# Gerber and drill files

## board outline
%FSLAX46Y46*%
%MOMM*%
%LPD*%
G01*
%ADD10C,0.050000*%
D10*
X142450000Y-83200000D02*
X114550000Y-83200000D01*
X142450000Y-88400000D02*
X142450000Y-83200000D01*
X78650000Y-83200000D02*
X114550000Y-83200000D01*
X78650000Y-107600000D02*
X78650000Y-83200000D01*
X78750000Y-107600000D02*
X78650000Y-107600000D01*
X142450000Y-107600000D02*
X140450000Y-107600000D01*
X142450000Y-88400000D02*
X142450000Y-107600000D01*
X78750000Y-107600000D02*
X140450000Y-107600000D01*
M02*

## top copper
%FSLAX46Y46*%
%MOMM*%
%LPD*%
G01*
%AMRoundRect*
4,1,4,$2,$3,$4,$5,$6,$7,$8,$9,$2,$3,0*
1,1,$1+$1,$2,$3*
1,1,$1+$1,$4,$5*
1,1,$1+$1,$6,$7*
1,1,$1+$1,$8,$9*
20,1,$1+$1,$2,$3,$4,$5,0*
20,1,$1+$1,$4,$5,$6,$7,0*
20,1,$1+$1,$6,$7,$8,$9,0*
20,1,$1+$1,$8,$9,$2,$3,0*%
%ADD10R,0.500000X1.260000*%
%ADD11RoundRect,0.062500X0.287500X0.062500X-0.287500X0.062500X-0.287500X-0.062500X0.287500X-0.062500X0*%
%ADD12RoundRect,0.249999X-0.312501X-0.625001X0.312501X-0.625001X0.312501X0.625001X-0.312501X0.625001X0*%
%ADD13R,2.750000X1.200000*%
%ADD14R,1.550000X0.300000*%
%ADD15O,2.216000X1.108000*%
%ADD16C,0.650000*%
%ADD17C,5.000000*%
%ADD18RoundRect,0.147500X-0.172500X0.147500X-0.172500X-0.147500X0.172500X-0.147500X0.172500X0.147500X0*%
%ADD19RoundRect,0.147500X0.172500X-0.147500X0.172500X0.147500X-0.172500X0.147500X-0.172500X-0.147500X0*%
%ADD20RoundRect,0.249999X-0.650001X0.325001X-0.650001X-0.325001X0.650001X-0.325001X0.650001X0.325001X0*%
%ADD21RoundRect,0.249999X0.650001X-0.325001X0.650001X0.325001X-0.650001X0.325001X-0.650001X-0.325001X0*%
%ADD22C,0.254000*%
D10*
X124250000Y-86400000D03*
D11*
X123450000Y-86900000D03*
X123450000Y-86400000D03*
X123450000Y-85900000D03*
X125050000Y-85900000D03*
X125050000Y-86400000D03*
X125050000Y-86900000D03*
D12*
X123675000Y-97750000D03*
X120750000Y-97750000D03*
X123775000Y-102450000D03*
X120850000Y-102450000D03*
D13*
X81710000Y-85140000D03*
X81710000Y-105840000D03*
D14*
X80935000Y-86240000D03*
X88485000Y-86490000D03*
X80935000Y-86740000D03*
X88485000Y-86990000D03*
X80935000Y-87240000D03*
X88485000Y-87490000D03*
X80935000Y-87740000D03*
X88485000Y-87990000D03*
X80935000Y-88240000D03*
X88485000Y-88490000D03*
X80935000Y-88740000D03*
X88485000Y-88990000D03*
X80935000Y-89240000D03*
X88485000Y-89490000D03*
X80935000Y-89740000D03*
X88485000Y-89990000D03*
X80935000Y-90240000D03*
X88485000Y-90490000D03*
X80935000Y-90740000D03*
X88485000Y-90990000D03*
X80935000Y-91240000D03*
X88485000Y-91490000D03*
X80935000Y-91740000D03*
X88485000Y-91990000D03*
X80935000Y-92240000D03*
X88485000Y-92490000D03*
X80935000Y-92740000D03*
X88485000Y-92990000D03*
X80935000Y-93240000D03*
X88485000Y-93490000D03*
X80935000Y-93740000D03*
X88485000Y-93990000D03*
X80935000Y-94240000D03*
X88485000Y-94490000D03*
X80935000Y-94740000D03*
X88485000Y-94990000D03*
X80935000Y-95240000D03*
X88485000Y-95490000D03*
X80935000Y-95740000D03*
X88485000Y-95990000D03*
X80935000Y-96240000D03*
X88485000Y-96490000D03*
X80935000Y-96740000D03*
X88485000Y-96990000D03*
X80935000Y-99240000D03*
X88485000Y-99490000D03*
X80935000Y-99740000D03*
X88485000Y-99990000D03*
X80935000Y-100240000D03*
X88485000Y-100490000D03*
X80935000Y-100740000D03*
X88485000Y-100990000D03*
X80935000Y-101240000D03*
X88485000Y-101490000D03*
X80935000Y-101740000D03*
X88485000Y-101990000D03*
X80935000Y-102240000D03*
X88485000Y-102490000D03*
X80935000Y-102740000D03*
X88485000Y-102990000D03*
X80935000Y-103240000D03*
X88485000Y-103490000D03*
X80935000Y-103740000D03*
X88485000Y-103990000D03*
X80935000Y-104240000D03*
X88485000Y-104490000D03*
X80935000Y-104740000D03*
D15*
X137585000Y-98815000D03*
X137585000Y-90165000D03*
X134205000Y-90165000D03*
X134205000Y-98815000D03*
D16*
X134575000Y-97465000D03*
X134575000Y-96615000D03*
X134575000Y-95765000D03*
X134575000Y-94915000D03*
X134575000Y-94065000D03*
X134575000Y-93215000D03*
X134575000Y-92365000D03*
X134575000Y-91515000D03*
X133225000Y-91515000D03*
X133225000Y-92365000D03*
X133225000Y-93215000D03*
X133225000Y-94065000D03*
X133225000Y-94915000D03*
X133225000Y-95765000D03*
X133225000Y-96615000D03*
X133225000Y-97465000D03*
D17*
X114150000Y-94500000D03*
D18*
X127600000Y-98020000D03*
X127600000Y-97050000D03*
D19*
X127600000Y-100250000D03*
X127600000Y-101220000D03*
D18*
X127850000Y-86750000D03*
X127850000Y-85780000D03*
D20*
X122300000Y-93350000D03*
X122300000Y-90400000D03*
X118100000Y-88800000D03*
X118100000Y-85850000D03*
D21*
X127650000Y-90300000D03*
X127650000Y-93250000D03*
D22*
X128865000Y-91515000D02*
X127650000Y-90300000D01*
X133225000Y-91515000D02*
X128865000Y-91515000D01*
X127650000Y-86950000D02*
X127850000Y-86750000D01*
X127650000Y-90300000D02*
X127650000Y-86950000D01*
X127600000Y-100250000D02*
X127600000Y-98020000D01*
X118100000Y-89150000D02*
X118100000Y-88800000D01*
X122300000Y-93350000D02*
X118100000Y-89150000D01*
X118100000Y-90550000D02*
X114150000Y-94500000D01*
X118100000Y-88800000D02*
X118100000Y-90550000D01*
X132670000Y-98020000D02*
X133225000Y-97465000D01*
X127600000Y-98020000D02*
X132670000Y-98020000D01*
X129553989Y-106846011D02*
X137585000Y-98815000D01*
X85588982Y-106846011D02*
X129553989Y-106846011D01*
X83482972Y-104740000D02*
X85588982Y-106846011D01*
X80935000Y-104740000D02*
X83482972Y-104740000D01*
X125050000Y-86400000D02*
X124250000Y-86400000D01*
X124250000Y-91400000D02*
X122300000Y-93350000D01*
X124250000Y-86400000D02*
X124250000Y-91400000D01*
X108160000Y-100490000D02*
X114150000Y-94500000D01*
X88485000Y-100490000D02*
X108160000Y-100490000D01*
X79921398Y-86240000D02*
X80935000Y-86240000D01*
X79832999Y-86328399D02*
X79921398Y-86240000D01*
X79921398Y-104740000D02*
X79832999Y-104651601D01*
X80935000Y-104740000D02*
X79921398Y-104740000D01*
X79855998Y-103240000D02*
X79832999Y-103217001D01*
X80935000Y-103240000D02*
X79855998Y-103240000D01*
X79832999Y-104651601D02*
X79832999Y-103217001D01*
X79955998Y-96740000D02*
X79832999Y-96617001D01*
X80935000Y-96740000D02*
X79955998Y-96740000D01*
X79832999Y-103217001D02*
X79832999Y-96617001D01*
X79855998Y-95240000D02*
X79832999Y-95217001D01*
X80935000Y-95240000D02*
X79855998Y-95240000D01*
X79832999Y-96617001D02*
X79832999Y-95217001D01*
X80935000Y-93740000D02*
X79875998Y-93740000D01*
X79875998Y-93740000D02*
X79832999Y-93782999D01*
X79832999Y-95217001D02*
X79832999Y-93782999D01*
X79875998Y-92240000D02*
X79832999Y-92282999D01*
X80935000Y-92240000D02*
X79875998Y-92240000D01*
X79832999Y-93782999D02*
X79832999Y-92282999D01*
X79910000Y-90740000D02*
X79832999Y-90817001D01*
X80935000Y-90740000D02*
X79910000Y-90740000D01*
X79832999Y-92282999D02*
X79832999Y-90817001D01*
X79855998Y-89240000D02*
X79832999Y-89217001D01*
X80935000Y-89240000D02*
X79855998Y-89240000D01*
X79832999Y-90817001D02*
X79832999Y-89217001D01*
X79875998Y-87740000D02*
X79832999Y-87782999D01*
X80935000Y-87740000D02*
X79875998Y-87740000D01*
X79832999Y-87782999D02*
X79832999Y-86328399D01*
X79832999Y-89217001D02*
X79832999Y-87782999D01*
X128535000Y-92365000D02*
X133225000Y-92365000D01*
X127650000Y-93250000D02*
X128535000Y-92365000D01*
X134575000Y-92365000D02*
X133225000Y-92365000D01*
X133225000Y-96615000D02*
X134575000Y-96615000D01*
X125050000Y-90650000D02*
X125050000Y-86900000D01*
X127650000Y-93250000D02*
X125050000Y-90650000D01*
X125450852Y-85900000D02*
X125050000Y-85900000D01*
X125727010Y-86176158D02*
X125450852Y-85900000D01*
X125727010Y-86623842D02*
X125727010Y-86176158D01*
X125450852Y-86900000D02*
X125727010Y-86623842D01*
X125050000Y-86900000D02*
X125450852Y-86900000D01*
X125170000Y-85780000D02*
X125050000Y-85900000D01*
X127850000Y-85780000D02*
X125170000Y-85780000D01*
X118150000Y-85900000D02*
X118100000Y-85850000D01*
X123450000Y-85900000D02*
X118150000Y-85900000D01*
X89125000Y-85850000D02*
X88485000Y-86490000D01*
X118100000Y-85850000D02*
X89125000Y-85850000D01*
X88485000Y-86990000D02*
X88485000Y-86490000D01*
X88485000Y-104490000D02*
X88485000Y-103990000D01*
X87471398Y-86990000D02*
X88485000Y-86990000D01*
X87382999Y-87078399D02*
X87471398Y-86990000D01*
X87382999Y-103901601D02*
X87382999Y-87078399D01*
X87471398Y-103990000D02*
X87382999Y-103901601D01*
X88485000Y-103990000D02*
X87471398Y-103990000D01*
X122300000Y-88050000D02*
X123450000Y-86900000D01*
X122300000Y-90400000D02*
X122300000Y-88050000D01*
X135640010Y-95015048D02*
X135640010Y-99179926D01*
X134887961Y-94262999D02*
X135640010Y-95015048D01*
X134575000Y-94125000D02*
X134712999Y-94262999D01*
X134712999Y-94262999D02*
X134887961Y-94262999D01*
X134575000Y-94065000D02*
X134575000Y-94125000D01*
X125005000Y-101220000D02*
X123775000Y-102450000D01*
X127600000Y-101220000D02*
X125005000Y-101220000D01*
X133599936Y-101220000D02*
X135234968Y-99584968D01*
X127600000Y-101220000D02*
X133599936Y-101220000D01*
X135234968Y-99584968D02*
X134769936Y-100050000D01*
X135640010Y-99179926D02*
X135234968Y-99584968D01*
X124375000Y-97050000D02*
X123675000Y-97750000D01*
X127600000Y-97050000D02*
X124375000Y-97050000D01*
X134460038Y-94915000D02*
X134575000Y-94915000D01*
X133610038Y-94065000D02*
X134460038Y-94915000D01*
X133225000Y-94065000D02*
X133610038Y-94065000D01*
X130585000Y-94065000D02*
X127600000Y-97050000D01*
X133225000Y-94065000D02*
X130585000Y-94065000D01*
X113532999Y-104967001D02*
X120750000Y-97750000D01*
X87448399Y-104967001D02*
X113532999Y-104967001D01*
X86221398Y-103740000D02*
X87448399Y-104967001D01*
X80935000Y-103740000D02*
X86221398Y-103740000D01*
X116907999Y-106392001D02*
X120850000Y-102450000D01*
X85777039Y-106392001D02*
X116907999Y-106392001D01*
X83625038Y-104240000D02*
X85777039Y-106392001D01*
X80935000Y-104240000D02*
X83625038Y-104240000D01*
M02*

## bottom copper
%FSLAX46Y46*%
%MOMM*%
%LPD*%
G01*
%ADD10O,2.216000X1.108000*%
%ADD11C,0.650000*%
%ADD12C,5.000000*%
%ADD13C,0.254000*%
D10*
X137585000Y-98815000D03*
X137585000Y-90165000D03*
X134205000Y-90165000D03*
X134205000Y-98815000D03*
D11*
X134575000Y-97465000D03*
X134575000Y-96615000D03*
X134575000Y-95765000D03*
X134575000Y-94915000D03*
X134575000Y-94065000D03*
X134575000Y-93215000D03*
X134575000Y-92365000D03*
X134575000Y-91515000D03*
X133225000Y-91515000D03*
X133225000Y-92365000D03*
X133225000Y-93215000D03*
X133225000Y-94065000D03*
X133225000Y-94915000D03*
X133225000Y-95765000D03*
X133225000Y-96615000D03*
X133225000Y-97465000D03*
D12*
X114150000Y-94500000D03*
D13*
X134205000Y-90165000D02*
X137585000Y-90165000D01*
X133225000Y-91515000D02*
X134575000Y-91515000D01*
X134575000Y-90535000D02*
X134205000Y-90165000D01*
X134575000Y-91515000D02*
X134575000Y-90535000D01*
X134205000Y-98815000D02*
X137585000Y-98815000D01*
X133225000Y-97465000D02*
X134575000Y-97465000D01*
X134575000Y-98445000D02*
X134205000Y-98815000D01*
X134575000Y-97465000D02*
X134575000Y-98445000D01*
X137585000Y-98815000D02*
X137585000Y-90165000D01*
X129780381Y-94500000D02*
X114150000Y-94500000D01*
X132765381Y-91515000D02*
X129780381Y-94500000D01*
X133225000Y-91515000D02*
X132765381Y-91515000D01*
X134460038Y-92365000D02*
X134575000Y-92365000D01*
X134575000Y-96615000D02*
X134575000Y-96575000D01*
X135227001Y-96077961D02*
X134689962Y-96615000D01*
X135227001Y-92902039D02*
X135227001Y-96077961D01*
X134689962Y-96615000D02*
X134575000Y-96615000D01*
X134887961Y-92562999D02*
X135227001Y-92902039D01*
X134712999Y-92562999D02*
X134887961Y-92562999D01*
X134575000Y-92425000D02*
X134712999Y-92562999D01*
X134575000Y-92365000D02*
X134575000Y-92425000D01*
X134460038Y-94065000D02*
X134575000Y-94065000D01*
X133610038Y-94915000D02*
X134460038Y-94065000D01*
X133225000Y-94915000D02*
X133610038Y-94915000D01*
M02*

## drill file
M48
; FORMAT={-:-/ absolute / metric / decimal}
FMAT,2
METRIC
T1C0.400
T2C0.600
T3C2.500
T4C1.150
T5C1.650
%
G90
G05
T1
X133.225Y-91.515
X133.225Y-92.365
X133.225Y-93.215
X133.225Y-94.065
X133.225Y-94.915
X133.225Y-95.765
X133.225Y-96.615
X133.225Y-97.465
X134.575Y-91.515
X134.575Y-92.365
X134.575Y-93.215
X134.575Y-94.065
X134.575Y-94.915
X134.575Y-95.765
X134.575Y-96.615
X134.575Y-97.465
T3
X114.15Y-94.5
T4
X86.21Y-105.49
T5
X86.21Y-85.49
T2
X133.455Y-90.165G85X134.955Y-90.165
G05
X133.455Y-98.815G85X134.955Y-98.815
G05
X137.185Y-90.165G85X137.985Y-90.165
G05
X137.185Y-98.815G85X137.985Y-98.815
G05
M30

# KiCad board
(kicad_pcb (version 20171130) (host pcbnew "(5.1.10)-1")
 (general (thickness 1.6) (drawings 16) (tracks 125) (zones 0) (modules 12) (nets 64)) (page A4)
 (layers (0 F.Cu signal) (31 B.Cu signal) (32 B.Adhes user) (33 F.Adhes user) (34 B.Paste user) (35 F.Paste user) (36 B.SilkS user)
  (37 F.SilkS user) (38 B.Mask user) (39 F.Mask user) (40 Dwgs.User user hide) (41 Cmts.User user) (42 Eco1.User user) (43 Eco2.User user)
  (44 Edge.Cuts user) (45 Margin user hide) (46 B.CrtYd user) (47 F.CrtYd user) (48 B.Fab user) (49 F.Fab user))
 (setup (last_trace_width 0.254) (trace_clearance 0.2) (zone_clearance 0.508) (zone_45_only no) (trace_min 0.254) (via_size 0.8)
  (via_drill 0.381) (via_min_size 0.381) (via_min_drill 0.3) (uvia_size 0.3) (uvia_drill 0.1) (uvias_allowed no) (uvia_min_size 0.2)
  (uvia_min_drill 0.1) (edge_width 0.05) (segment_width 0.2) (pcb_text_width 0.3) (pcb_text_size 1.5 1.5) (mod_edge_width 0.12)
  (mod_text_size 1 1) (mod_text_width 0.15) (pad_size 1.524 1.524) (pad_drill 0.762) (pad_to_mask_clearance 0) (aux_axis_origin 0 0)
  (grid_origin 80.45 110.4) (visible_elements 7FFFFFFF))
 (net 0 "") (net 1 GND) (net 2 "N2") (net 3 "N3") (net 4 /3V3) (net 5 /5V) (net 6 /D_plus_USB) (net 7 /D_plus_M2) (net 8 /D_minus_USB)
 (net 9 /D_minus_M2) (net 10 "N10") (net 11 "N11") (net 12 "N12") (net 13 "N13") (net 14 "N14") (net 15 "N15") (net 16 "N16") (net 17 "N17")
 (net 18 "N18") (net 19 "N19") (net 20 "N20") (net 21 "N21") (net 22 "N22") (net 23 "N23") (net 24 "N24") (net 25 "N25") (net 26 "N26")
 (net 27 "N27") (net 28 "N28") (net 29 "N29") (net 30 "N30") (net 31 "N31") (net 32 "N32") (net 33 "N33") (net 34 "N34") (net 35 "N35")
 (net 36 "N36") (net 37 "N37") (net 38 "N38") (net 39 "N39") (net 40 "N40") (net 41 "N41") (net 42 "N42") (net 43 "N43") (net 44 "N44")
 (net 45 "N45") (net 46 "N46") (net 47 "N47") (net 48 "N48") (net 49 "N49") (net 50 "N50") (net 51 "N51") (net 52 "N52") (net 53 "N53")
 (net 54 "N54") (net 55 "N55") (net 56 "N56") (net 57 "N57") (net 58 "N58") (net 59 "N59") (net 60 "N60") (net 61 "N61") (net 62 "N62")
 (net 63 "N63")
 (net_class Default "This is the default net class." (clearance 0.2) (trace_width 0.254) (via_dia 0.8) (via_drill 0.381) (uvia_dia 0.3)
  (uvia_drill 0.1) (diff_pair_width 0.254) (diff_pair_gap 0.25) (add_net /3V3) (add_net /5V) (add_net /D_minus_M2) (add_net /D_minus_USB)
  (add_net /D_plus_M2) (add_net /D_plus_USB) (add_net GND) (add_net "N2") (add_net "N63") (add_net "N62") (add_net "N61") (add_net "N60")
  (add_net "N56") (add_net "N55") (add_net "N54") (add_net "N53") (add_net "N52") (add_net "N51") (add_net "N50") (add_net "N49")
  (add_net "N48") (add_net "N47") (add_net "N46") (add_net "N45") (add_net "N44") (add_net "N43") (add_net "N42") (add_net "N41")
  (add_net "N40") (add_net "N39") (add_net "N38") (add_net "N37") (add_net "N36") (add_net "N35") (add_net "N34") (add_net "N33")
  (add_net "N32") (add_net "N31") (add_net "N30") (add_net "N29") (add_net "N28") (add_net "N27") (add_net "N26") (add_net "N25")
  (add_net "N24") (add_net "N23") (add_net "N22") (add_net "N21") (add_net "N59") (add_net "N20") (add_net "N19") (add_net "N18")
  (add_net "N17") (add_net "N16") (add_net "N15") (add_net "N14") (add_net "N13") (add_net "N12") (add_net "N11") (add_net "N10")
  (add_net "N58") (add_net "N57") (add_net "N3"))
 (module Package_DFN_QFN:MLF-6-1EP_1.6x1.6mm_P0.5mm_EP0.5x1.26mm (layer F.Cu) (at 124.25 86.4 180)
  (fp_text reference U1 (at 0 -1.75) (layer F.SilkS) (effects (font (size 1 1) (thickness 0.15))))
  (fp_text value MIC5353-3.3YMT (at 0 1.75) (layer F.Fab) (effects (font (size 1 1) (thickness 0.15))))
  (pad "" smd roundrect (at 0 0.315 180) (size 0.4 0.51) (layers F.Paste) (roundrect_rratio 0.25))
  (pad "" smd roundrect (at 0 -0.315 180) (size 0.4 0.51) (layers F.Paste) (roundrect_rratio 0.25))
  (pad 7 smd rect (at 0 0 180) (size 0.5 1.26) (layers F.Cu F.Mask) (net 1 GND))
  (pad 6 smd roundrect (at 0.8 -0.5 180) (size 0.7 0.25) (layers F.Cu F.Paste F.Mask) (roundrect_rratio 0.25) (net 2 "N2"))
  (pad 5 smd roundrect (at 0.8 0 180) (size 0.7 0.25) (layers F.Cu F.Paste F.Mask) (roundrect_rratio 0.25) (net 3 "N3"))
  (pad 4 smd roundrect (at 0.8 0.5 180) (size 0.7 0.25) (layers F.Cu F.Paste F.Mask) (roundrect_rratio 0.25) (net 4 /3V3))
  (pad 3 smd roundrect (at -0.8 0.5 180) (size 0.7 0.25) (layers F.Cu F.Paste F.Mask) (roundrect_rratio 0.25) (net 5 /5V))
  (pad 2 smd roundrect (at -0.8 0 180) (size 0.7 0.25) (layers F.Cu F.Paste F.Mask) (roundrect_rratio 0.25) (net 1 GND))
  (pad 1 smd roundrect (at -0.8 -0.5 180) (size 0.7 0.25) (layers F.Cu F.Paste F.Mask) (roundrect_rratio 0.25) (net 5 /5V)))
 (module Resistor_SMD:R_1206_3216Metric (layer F.Cu) (at 122.2125 97.75)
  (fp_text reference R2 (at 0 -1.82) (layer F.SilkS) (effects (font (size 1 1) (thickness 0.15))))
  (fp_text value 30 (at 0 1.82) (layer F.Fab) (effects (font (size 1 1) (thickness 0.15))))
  (pad 2 smd roundrect (at 1.4625 0) (size 1.125 1.75) (layers F.Cu F.Paste F.Mask) (roundrect_rratio 0.2222213333333333)
   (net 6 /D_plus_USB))
  (pad 1 smd roundrect (at -1.4625 0) (size 1.125 1.75) (layers F.Cu F.Paste F.Mask) (roundrect_rratio 0.2222213333333333)
   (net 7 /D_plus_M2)))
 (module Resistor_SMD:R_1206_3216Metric (layer F.Cu) (at 122.3125 102.45)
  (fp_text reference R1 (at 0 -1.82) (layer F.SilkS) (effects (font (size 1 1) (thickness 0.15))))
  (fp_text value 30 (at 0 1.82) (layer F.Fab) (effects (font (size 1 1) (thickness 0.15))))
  (pad 2 smd roundrect (at 1.4625 0) (size 1.125 1.75) (layers F.Cu F.Paste F.Mask) (roundrect_rratio 0.2222213333333333)
   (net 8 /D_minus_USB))
  (pad 1 smd roundrect (at -1.4625 0) (size 1.125 1.75) (layers F.Cu F.Paste F.Mask) (roundrect_rratio 0.2222213333333333)
   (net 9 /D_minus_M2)))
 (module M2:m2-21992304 (layer F.Cu) (at 84.56 95.49 90)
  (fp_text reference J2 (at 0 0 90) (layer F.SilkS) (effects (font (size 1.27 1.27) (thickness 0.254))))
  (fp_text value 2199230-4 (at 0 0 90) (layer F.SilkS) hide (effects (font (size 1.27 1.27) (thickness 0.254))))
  (pad MP2 smd rect (at 10.35 -2.85 90) (size 1.2 2.75) (layers F.Cu F.Paste F.Mask))
  (pad MP1 smd rect (at -10.35 -2.85 90) (size 1.2 2.75) (layers F.Cu F.Paste F.Mask))
  (pad MH2 np_thru_hole circle (at 10 1.65 90) (size 1.65 0) (drill 1.65) (layers *.Cu *.Mask))
  (pad MH1 np_thru_hole circle (at -10 1.65 90) (size 1.15 0) (drill 1.15) (layers *.Cu *.Mask))
  (pad 75 smd rect (at 9.25 -3.625 90) (size 0.3 1.55) (layers F.Cu F.Paste F.Mask) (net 1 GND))
  (pad 74 smd rect (at 9 3.925 90) (size 0.3 1.55) (layers F.Cu F.Paste F.Mask) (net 4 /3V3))
  (pad 73 smd rect (at 8.75 -3.625 90) (size 0.3 1.55) (layers F.Cu F.Paste F.Mask) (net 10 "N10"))
  (pad 72 smd rect (at 8.5 3.925 90) (size 0.3 1.55) (layers F.Cu F.Paste F.Mask) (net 4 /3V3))
  (pad 71 smd rect (at 8.25 -3.625 90) (size 0.3 1.55) (layers F.Cu F.Paste F.Mask) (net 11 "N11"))
  (pad 70 smd rect (at 8 3.925 90) (size 0.3 1.55) (layers F.Cu F.Paste F.Mask) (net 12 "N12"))
  (pad 69 smd rect (at 7.75 -3.625 90) (size 0.3 1.55) (layers F.Cu F.Paste F.Mask) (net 1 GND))
  (pad 68 smd rect (at 7.5 3.925 90) (size 0.3 1.55) (layers F.Cu F.Paste F.Mask) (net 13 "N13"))
  (pad 67 smd rect (at 7.25 -3.625 90) (size 0.3 1.55) (layers F.Cu F.Paste F.Mask) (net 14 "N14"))
  (pad 66 smd rect (at 7 3.925 90) (size 0.3 1.55) (layers F.Cu F.Paste F.Mask) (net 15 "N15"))
  (pad 65 smd rect (at 6.75 -3.625 90) (size 0.3 1.55) (layers F.Cu F.Paste F.Mask) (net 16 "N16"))
  (pad 64 smd rect (at 6.5 3.925 90) (size 0.3 1.55) (layers F.Cu F.Paste F.Mask) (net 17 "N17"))
  (pad 63 smd rect (at 6.25 -3.625 90) (size 0.3 1.55) (layers F.Cu F.Paste F.Mask) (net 1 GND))
  (pad 62 smd rect (at 6 3.925 90) (size 0.3 1.55) (layers F.Cu F.Paste F.Mask) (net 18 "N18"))
  (pad 61 smd rect (at 5.75 -3.625 90) (size 0.3 1.55) (layers F.Cu F.Paste F.Mask) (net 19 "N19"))
  (pad 60 smd rect (at 5.5 3.925 90) (size 0.3 1.55) (layers F.Cu F.Paste F.Mask) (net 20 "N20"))
  (pad 59 smd rect (at 5.25 -3.625 90) (size 0.3 1.55) (layers F.Cu F.Paste F.Mask) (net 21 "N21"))
  (pad 58 smd rect (at 5 3.925 90) (size 0.3 1.55) (layers F.Cu F.Paste F.Mask) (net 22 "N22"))
  (pad 57 smd rect (at 4.75 -3.625 90) (size 0.3 1.55) (layers F.Cu F.Paste F.Mask) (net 1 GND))
  (pad 56 smd rect (at 4.5 3.925 90) (size 0.3 1.55) (layers F.Cu F.Paste F.Mask) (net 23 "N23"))
  (pad 55 smd rect (at 4.25 -3.625 90) (size 0.3 1.55) (layers F.Cu F.Paste F.Mask) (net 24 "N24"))
  (pad 54 smd rect (at 4 3.925 90) (size 0.3 1.55) (layers F.Cu F.Paste F.Mask) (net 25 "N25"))
  (pad 53 smd rect (at 3.75 -3.625 90) (size 0.3 1.55) (layers F.Cu F.Paste F.Mask) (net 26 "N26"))
  (pad 52 smd rect (at 3.5 3.925 90) (size 0.3 1.55) (layers F.Cu F.Paste F.Mask) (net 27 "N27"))
  (pad 51 smd rect (at 3.25 -3.625 90) (size 0.3 1.55) (layers F.Cu F.Paste F.Mask) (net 1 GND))
  (pad 50 smd rect (at 3 3.925 90) (size 0.3 1.55) (layers F.Cu F.Paste F.Mask) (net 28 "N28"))
  (pad 49 smd rect (at 2.75 -3.625 90) (size 0.3 1.55) (layers F.Cu F.Paste F.Mask) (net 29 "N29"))
  (pad 48 smd rect (at 2.5 3.925 90) (size 0.3 1.55) (layers F.Cu F.Paste F.Mask) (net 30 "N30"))
  (pad 47 smd rect (at 2.25 -3.625 90) (size 0.3 1.55) (layers F.Cu F.Paste F.Mask) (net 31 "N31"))
  (pad 46 smd rect (at 2 3.925 90) (size 0.3 1.55) (layers F.Cu F.Paste F.Mask) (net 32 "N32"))
  (pad 45 smd rect (at 1.75 -3.625 90) (size 0.3 1.55) (layers F.Cu F.Paste F.Mask) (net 1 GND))
  (pad 44 smd rect (at 1.5 3.925 90) (size 0.3 1.55) (layers F.Cu F.Paste F.Mask) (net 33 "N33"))
  (pad 43 smd rect (at 1.25 -3.625 90) (size 0.3 1.55) (layers F.Cu F.Paste F.Mask) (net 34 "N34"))
  (pad 42 smd rect (at 1 3.925 90) (size 0.3 1.55) (layers F.Cu F.Paste F.Mask) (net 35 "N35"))
  (pad 41 smd rect (at 0.75 -3.625 90) (size 0.3 1.55) (layers F.Cu F.Paste F.Mask) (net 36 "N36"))
  (pad 40 smd rect (at 0.5 3.925 90) (size 0.3 1.55) (layers F.Cu F.Paste F.Mask) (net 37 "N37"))
  (pad 39 smd rect (at 0.25 -3.625 90) (size 0.3 1.55) (layers F.Cu F.Paste F.Mask) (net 1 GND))
  (pad 38 smd rect (at 0 3.925 90) (size 0.3 1.55) (layers F.Cu F.Paste F.Mask) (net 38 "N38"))
  (pad 37 smd rect (at -0.25 -3.625 90) (size 0.3 1.55) (layers F.Cu F.Paste F.Mask) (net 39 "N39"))
  (pad 36 smd rect (at -0.5 3.925 90) (size 0.3 1.55) (layers F.Cu F.Paste F.Mask) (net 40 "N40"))
  (pad 35 smd rect (at -0.75 -3.625 90) (size 0.3 1.55) (layers F.Cu F.Paste F.Mask) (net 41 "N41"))
  (pad 34 smd rect (at -1 3.925 90) (size 0.3 1.55) (layers F.Cu F.Paste F.Mask) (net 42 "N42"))
  (pad 33 smd rect (at -1.25 -3.625 90) (size 0.3 1.55) (layers F.Cu F.Paste F.Mask) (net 1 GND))
  (pad 32 smd rect (at -1.5 3.925 90) (size 0.3 1.55) (layers F.Cu F.Paste F.Mask) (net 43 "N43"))
  (pad 23 smd rect (at -3.75 -3.625 90) (size 0.3 1.55) (layers F.Cu F.Paste F.Mask) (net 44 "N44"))
  (pad 22 smd rect (at -4 3.925 90) (size 0.3 1.55) (layers F.Cu F.Paste F.Mask) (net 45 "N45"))
  (pad 21 smd rect (at -4.25 -3.625 90) (size 0.3 1.55) (layers F.Cu F.Paste F.Mask) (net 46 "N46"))
  (pad 20 smd rect (at -4.5 3.925 90) (size 0.3 1.55) (layers F.Cu F.Paste F.Mask) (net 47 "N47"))
  (pad 19 smd rect (at -4.75 -3.625 90) (size 0.3 1.55) (layers F.Cu F.Paste F.Mask) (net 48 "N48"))
  (pad 18 smd rect (at -5 3.925 90) (size 0.3 1.55) (layers F.Cu F.Paste F.Mask) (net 1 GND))
  (pad 17 smd rect (at -5.25 -3.625 90) (size 0.3 1.55) (layers F.Cu F.Paste F.Mask) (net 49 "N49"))
  (pad 16 smd rect (at -5.5 3.925 90) (size 0.3 1.55) (layers F.Cu F.Paste F.Mask) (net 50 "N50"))
  (pad 15 smd rect (at -5.75 -3.625 90) (size 0.3 1.55) (layers F.Cu F.Paste F.Mask) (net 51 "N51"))
  (pad 14 smd rect (at -6 3.925 90) (size 0.3 1.55) (layers F.Cu F.Paste F.Mask) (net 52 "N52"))
  (pad 13 smd rect (at -6.25 -3.625 90) (size 0.3 1.55) (layers F.Cu F.Paste F.Mask) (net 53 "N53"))
  (pad 12 smd rect (at -6.5 3.925 90) (size 0.3 1.55) (layers F.Cu F.Paste F.Mask) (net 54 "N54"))
  (pad 11 smd rect (at -6.75 -3.625 90) (size 0.3 1.55) (layers F.Cu F.Paste F.Mask) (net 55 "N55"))
  (pad 10 smd rect (at -7 3.925 90) (size 0.3 1.55) (layers F.Cu F.Paste F.Mask) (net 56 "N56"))
  (pad 9 smd rect (at -7.25 -3.625 90) (size 0.3 1.55) (layers F.Cu F.Paste F.Mask) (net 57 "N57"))
  (pad 8 smd rect (at -7.5 3.925 90) (size 0.3 1.55) (layers F.Cu F.Paste F.Mask) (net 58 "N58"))
  (pad 7 smd rect (at -7.75 -3.625 90) (size 0.3 1.55) (layers F.Cu F.Paste F.Mask) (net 1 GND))
  (pad 6 smd rect (at -8 3.925 90) (size 0.3 1.55) (layers F.Cu F.Paste F.Mask) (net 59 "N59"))
  (pad 5 smd rect (at -8.25 -3.625 90) (size 0.3 1.55) (layers F.Cu F.Paste F.Mask) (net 7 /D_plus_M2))
  (pad 4 smd rect (at -8.5 3.925 90) (size 0.3 1.55) (layers F.Cu F.Paste F.Mask) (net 4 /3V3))
  (pad 3 smd rect (at -8.75 -3.625 90) (size 0.3 1.55) (layers F.Cu F.Paste F.Mask) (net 9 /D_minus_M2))
  (pad 2 smd rect (at -9 3.925 90) (size 0.3 1.55) (layers F.Cu F.Paste F.Mask) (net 4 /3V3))
  (pad 1 smd rect (at -9.25 -3.625 90) (size 0.3 1.55) (layers F.Cu F.Paste F.Mask) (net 1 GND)))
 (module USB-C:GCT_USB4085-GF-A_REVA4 (layer F.Cu) (at 137.25 94.49 90)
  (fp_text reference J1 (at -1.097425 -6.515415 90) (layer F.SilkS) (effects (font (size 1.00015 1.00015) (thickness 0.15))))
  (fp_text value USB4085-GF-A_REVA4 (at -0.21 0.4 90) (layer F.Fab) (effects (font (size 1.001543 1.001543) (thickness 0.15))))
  (pad P4 thru_hole oval (at -4.325 0.335 90) (size 1.108 2.216) (drill oval 0.6 1.4) (layers *.Cu *.Mask) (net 1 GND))
  (pad P3 thru_hole oval (at 4.325 0.335 90) (size 1.108 2.216) (drill oval 0.6 1.4) (layers *.Cu *.Mask) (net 1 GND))
  (pad P2 thru_hole oval (at 4.325 -3.045 90) (size 1.108 2.216) (drill oval 0.6 2.1) (layers *.Cu *.Mask) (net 1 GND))
  (pad P1 thru_hole oval (at -4.325 -3.045 90) (size 1.108 2.216) (drill oval 0.6 2.1) (layers *.Cu *.Mask) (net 1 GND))
  (pad B12 thru_hole circle (at -2.975 -2.675 90) (size 0.65 0.65) (drill 0.4) (layers *.Cu *.Mask) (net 1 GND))
  (pad B9 thru_hole circle (at -2.125 -2.675 90) (size 0.65 0.65) (drill 0.4) (layers *.Cu *.Mask) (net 5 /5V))
  (pad B8 thru_hole circle (at -1.275 -2.675 90) (size 0.65 0.65) (drill 0.4) (layers *.Cu *.Mask) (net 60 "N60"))
  (pad B7 thru_hole circle (at -0.425 -2.675 90) (size 0.65 0.65) (drill 0.4) (layers *.Cu *.Mask) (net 6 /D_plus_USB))
  (pad B6 thru_hole circle (at 0.425 -2.675 90) (size 0.65 0.65) (drill 0.4) (layers *.Cu *.Mask) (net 8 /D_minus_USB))
  (pad B5 thru_hole circle (at 1.275 -2.675 90) (size 0.65 0.65) (drill 0.4) (layers *.Cu *.Mask) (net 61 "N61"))
  (pad B4 thru_hole circle (at 2.125 -2.675 90) (size 0.65 0.65) (drill 0.4) (layers *.Cu *.Mask) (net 5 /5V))
  (pad B1 thru_hole circle (at 2.975 -2.675 90) (size 0.65 0.65) (drill 0.4) (layers *.Cu *.Mask) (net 1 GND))
  (pad A12 thru_hole circle (at 2.975 -4.025 90) (size 0.65 0.65) (drill 0.4) (layers *.Cu *.Mask) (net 1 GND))
  (pad A9 thru_hole circle (at 2.125 -4.025 90) (size 0.65 0.65) (drill 0.4) (layers *.Cu *.Mask) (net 5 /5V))
  (pad A8 thru_hole circle (at 1.275 -4.025 90) (size 0.65 0.65) (drill 0.4) (layers *.Cu *.Mask) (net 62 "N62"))
  (pad A7 thru_hole circle (at 0.425 -4.025 90) (size 0.65 0.65) (drill 0.4) (layers *.Cu *.Mask) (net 6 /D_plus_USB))
  (pad A6 thru_hole circle (at -0.425 -4.025 90) (size 0.65 0.65) (drill 0.4) (layers *.Cu *.Mask) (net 8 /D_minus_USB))
  (pad A5 thru_hole circle (at -1.275 -4.025 90) (size 0.65 0.65) (drill 0.4) (layers *.Cu *.Mask) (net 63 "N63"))
  (pad A4 thru_hole circle (at -2.125 -4.025 90) (size 0.65 0.65) (drill 0.4) (layers *.Cu *.Mask) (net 5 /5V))
  (pad A1 thru_hole circle (at -2.975 -4.025 90) (size 0.65 0.65) (drill 0.4) (layers *.Cu *.Mask) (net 1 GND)))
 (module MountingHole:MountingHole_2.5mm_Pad (layer F.Cu) (at 114.15 94.5)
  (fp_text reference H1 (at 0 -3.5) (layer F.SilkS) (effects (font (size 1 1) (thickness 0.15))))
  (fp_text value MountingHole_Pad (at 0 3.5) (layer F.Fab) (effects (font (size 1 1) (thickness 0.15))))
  (pad 1 thru_hole circle (at 0 0) (size 5 5) (drill 2.5) (layers *.Cu *.Mask) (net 1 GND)))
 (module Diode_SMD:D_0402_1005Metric (layer F.Cu) (at 127.6 97.535 270)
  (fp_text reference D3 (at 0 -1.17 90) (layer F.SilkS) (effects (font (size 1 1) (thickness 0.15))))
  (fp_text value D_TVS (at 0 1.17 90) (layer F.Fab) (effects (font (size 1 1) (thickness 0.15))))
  (pad 2 smd roundrect (at 0.485 0 270) (size 0.59 0.64) (layers F.Cu F.Paste F.Mask) (roundrect_rratio 0.25) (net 1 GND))
  (pad 1 smd roundrect (at -0.485 0 270) (size 0.59 0.64) (layers F.Cu F.Paste F.Mask) (roundrect_rratio 0.25) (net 6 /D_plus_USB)))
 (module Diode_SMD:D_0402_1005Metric (layer F.Cu) (at 127.6 100.735 90)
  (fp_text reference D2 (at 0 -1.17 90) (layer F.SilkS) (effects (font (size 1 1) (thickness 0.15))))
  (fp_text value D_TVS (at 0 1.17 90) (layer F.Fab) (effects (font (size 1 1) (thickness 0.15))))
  (pad 2 smd roundrect (at 0.485 0 90) (size 0.59 0.64) (layers F.Cu F.Paste F.Mask) (roundrect_rratio 0.25) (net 1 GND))
  (pad 1 smd roundrect (at -0.485 0 90) (size 0.59 0.64) (layers F.Cu F.Paste F.Mask) (roundrect_rratio 0.25) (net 8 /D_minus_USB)))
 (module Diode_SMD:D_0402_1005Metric (layer F.Cu) (at 127.85 86.265 270)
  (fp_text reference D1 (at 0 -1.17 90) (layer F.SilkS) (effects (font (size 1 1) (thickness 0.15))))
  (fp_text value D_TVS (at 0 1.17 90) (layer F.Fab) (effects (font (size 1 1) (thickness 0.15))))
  (pad 2 smd roundrect (at 0.485 0 270) (size 0.59 0.64) (layers F.Cu F.Paste F.Mask) (roundrect_rratio 0.25) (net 1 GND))
  (pad 1 smd roundrect (at -0.485 0 270) (size 0.59 0.64) (layers F.Cu F.Paste F.Mask) (roundrect_rratio 0.25) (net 5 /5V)))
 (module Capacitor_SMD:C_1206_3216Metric (layer F.Cu) (at 122.3 91.875 270)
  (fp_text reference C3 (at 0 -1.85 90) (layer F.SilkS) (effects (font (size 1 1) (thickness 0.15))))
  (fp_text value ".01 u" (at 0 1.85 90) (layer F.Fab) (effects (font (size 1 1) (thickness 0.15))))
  (pad 2 smd roundrect (at 1.475 0 270) (size 1.15 1.8) (layers F.Cu F.Paste F.Mask) (roundrect_rratio 0.2173904347826087) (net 1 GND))
  (pad 1 smd roundrect (at -1.475 0 270) (size 1.15 1.8) (layers F.Cu F.Paste F.Mask) (roundrect_rratio 0.2173904347826087) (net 2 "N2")))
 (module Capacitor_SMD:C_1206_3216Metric (layer F.Cu) (at 118.1 87.325 270)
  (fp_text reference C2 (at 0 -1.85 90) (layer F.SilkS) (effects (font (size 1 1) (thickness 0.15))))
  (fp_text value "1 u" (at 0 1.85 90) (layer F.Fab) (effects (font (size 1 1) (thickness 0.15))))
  (pad 2 smd roundrect (at 1.475 0 270) (size 1.15 1.8) (layers F.Cu F.Paste F.Mask) (roundrect_rratio 0.2173904347826087) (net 1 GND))
  (pad 1 smd roundrect (at -1.475 0 270) (size 1.15 1.8) (layers F.Cu F.Paste F.Mask) (roundrect_rratio 0.2173904347826087) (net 4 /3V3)))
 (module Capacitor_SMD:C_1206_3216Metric (layer F.Cu) (at 127.65 91.775 90)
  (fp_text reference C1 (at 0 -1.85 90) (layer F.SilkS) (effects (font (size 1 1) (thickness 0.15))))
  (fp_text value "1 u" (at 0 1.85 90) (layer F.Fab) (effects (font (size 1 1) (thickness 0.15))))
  (pad 2 smd roundrect (at 1.475 0 90) (size 1.15 1.8) (layers F.Cu F.Paste F.Mask) (roundrect_rratio 0.2173904347826087) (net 1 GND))
  (pad 1 smd roundrect (at -1.475 0 90) (size 1.15 1.8) (layers F.Cu F.Paste F.Mask) (roundrect_rratio 0.2173904347826087) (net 5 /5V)))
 (gr_line (start 142.45 83.2) (end 114.55 83.2) (layer Edge.Cuts) (width 0.05))
 (gr_line (start 142.45 88.4) (end 142.45 83.2) (layer Edge.Cuts) (width 0.05))
 (gr_line (start 78.65 83.2) (end 114.55 83.2) (layer Edge.Cuts) (width 0.05))
 (gr_line (start 78.65 107.6) (end 78.65 83.2) (layer Edge.Cuts) (width 0.05))
 (gr_line (start 78.75 107.6) (end 78.65 107.6) (layer Edge.Cuts) (width 0.05))
 (gr_line (start 142.45 107.6) (end 140.45 107.6) (layer Edge.Cuts) (width 0.05))
 (gr_line (start 142.45 88.4) (end 142.45 107.6) (layer Edge.Cuts) (width 0.05))
 (gr_line (start 78.75 107.6) (end 140.45 107.6) (layer Edge.Cuts) (width 0.05))
 (segment (start 134.205 90.165) (end 137.585 90.165) (width 0.254) (layer B.Cu) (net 1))
 (segment (start 133.225 91.515) (end 134.575 91.515) (width 0.254) (layer B.Cu) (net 1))
 (segment (start 134.575 90.535) (end 134.205 90.165) (width 0.254) (layer B.Cu) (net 1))
 (segment (start 134.575 91.515) (end 134.575 90.535) (width 0.254) (layer B.Cu) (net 1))
 (segment (start 134.205 98.815) (end 137.585 98.815) (width 0.254) (layer B.Cu) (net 1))
 (segment (start 133.225 97.465) (end 134.575 97.465) (width 0.254) (layer B.Cu) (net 1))
 (segment (start 134.575 98.445) (end 134.205 98.815) (width 0.254) (layer B.Cu) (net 1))
 (segment (start 134.575 97.465) (end 134.575 98.445) (width 0.254) (layer B.Cu) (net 1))
 (segment (start 137.585 98.815) (end 137.585 90.165) (width 0.254) (layer B.Cu) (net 1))
 (segment (start 128.865 91.515) (end 127.65 90.3) (width 0.254) (layer F.Cu) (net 1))
 (segment (start 133.225 91.515) (end 128.865 91.515) (width 0.254) (layer F.Cu) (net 1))
 (segment (start 127.65 86.95) (end 127.85 86.75) (width 0.254) (layer F.Cu) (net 1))
 (segment (start 127.65 90.3) (end 127.65 86.95) (width 0.254) (layer F.Cu) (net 1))
 (segment (start 127.6 100.25) (end 127.6 98.02) (width 0.254) (layer F.Cu) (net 1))
 (segment (start 118.1 89.15) (end 118.1 88.8) (width 0.254) (layer F.Cu) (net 1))
 (segment (start 122.3 93.35) (end 118.1 89.15) (width 0.254) (layer F.Cu) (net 1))
 (segment (start 118.1 90.55) (end 114.15 94.5) (width 0.254) (layer F.Cu) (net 1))
 (segment (start 118.1 88.8) (end 118.1 90.55) (width 0.254) (layer F.Cu) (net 1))
 (segment (start 132.67 98.02) (end 133.225 97.465) (width 0.254) (layer F.Cu) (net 1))
 (segment (start 127.6 98.02) (end 132.67 98.02) (width 0.254) (layer F.Cu) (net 1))
 (segment (start 129.553989 106.846011) (end 137.585 98.815) (width 0.254) (layer F.Cu) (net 1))
 (segment (start 85.588982 106.846011) (end 129.553989 106.846011) (width 0.254) (layer F.Cu) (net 1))
 (segment (start 83.482972 104.74) (end 85.588982 106.846011) (width 0.254) (layer F.Cu) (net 1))
 (segment (start 80.935 104.74) (end 83.482972 104.74) (width 0.254) (layer F.Cu) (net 1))
 (segment (start 125.05 86.4) (end 124.25 86.4) (width 0.254) (layer F.Cu) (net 1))
 (segment (start 124.25 91.4) (end 122.3 93.35) (width 0.254) (layer F.Cu) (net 1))
 (segment (start 124.25 86.4) (end 124.25 91.4) (width 0.254) (layer F.Cu) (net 1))
 (segment (start 108.16 100.49) (end 114.15 94.5) (width 0.254) (layer F.Cu) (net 1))
 (segment (start 88.485 100.49) (end 108.16 100.49) (width 0.254) (layer F.Cu) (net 1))
 (segment (start 79.921398 86.24) (end 80.935 86.24) (width 0.254) (layer F.Cu) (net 1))
 (segment (start 79.832999 86.328399) (end 79.921398 86.24) (width 0.254) (layer F.Cu) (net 1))
 (segment (start 79.921398 104.74) (end 79.832999 104.651601) (width 0.254) (layer F.Cu) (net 1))
 (segment (start 80.935 104.74) (end 79.921398 104.74) (width 0.254) (layer F.Cu) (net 1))
 (segment (start 79.855998 103.24) (end 79.832999 103.217001) (width 0.254) (layer F.Cu) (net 1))
 (segment (start 80.935 103.24) (end 79.855998 103.24) (width 0.254) (layer F.Cu) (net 1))
 (segment (start 79.832999 104.651601) (end 79.832999 103.217001) (width 0.254) (layer F.Cu) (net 1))
 (segment (start 79.955998 96.74) (end 79.832999 96.617001) (width 0.254) (layer F.Cu) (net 1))
 (segment (start 80.935 96.74) (end 79.955998 96.74) (width 0.254) (layer F.Cu) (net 1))
 (segment (start 79.832999 103.217001) (end 79.832999 96.617001) (width 0.254) (layer F.Cu) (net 1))
 (segment (start 79.855998 95.24) (end 79.832999 95.217001) (width 0.254) (layer F.Cu) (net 1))
 (segment (start 80.935 95.24) (end 79.855998 95.24) (width 0.254) (layer F.Cu) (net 1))
 (segment (start 79.832999 96.617001) (end 79.832999 95.217001) (width 0.254) (layer F.Cu) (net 1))
 (segment (start 80.935 93.74) (end 79.875998 93.74) (width 0.254) (layer F.Cu) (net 1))
 (segment (start 79.875998 93.74) (end 79.832999 93.782999) (width 0.254) (layer F.Cu) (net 1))
 (segment (start 79.832999 95.217001) (end 79.832999 93.782999) (width 0.254) (layer F.Cu) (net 1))
 (segment (start 79.875998 92.24) (end 79.832999 92.282999) (width 0.254) (layer F.Cu) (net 1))
 (segment (start 80.935 92.24) (end 79.875998 92.24) (width 0.254) (layer F.Cu) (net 1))
 (segment (start 79.832999 93.782999) (end 79.832999 92.282999) (width 0.254) (layer F.Cu) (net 1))
 (segment (start 79.91 90.74) (end 79.832999 90.817001) (width 0.254) (layer F.Cu) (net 1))
 (segment (start 80.935 90.74) (end 79.91 90.74) (width 0.254) (layer F.Cu) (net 1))
 (segment (start 79.832999 92.282999) (end 79.832999 90.817001) (width 0.254) (layer F.Cu) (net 1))
 (segment (start 79.855998 89.24) (end 79.832999 89.217001) (width 0.254) (layer F.Cu) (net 1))
 (segment (start 80.935 89.24) (end 79.855998 89.24) (width 0.254) (layer F.Cu) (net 1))
 (segment (start 79.832999 90.817001) (end 79.832999 89.217001) (width 0.254) (layer F.Cu) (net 1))
 (segment (start 79.875998 87.74) (end 79.832999 87.782999) (width 0.254) (layer F.Cu) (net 1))
 (segment (start 80.935 87.74) (end 79.875998 87.74) (width 0.254) (layer F.Cu) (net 1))
 (segment (start 79.832999 87.782999) (end 79.832999 86.328399) (width 0.254) (layer F.Cu) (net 1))
 (segment (start 79.832999 89.217001) (end 79.832999 87.782999) (width 0.254) (layer F.Cu) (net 1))
 (segment (start 129.780381 94.5) (end 114.15 94.5) (width 0.254) (layer B.Cu) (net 1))
 (segment (start 132.765381 91.515) (end 129.780381 94.5) (width 0.254) (layer B.Cu) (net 1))
 (segment (start 133.225 91.515) (end 132.765381 91.515) (width 0.254) (layer B.Cu) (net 1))
 (segment (start 128.535 92.365) (end 133.225 92.365) (width 0.254) (layer F.Cu) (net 5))
 (segment (start 127.65 93.25) (end 128.535 92.365) (width 0.254) (layer F.Cu) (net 5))
 (segment (start 134.575 92.365) (end 133.225 92.365) (width 0.254) (layer F.Cu) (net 5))
 (segment (start 133.225 96.615) (end 134.575 96.615) (width 0.254) (layer F.Cu) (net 5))
 (segment (start 134.460038 92.365) (end 134.575 92.365) (width 0.254) (layer B.Cu) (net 5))
 (segment (start 134.575 96.615) (end 134.575 96.575) (width 0.254) (layer B.Cu) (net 5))
 (segment (start 125.05 90.65) (end 125.05 86.9) (width 0.254) (layer F.Cu) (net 5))
 (segment (start 127.65 93.25) (end 125.05 90.65) (width 0.254) (layer F.Cu) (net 5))
 (segment (start 125.450852 85.9) (end 125.05 85.9) (width 0.254) (layer F.Cu) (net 5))
 (segment (start 125.72701 86.176158) (end 125.450852 85.9) (width 0.254) (layer F.Cu) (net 5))
 (segment (start 125.72701 86.623842) (end 125.72701 86.176158) (width 0.254) (layer F.Cu) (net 5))
 (segment (start 125.450852 86.9) (end 125.72701 86.623842) (width 0.254) (layer F.Cu) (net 5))
 (segment (start 125.05 86.9) (end 125.450852 86.9) (width 0.254) (layer F.Cu) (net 5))
 (segment (start 125.17 85.78) (end 125.05 85.9) (width 0.254) (layer F.Cu) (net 5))
 (segment (start 127.85 85.78) (end 125.17 85.78) (width 0.254) (layer F.Cu) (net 5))
 (segment (start 135.227001 96.077961) (end 134.689962 96.615) (width 0.254) (layer B.Cu) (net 5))
 (segment (start 135.227001 92.902039) (end 135.227001 96.077961) (width 0.254) (layer B.Cu) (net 5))
 (segment (start 134.689962 96.615) (end 134.575 96.615) (width 0.254) (layer B.Cu) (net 5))
 (segment (start 134.887961 92.562999) (end 135.227001 92.902039) (width 0.254) (layer B.Cu) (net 5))
 (segment (start 134.712999 92.562999) (end 134.887961 92.562999) (width 0.254) (layer B.Cu) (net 5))
 (segment (start 134.575 92.425) (end 134.712999 92.562999) (width 0.254) (layer B.Cu) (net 5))
 (segment (start 134.575 92.365) (end 134.575 92.425) (width 0.254) (layer B.Cu) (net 5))
 (segment (start 118.15 85.9) (end 118.1 85.85) (width 0.254) (layer F.Cu) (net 4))
 (segment (start 123.45 85.9) (end 118.15 85.9) (width 0.254) (layer F.Cu) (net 4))
 (segment (start 89.125 85.85) (end 88.485 86.49) (width 0.254) (layer F.Cu) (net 4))
 (segment (start 118.1 85.85) (end 89.125 85.85) (width 0.254) (layer F.Cu) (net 4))
 (segment (start 88.485 86.99) (end 88.485 86.49) (width 0.254) (layer F.Cu) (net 4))
 (segment (start 88.485 104.49) (end 88.485 103.99) (width 0.254) (layer F.Cu) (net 4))
 (segment (start 87.471398 86.99) (end 88.485 86.99) (width 0.254) (layer F.Cu) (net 4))
 (segment (start 87.382999 87.078399) (end 87.471398 86.99) (width 0.254) (layer F.Cu) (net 4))
 (segment (start 87.382999 103.901601) (end 87.382999 87.078399) (width 0.254) (layer F.Cu) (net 4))
 (segment (start 87.471398 103.99) (end 87.382999 103.901601) (width 0.254) (layer F.Cu) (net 4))
 (segment (start 88.485 103.99) (end 87.471398 103.99) (width 0.254) (layer F.Cu) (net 4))
 (segment (start 122.3 88.05) (end 123.45 86.9) (width 0.254) (layer F.Cu) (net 2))
 (segment (start 122.3 90.4) (end 122.3 88.05) (width 0.254) (layer F.Cu) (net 2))
 (segment (start 134.460038 94.065) (end 134.575 94.065) (width 0.254) (layer B.Cu) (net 8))
 (segment (start 133.610038 94.915) (end 134.460038 94.065) (width 0.254) (layer B.Cu) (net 8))
 (segment (start 133.225 94.915) (end 133.610038 94.915) (width 0.254) (layer B.Cu) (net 8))
 (segment (start 135.64001 95.015048) (end 135.64001 99.179926) (width 0.254) (layer F.Cu) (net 8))
 (segment (start 134.887961 94.262999) (end 135.64001 95.015048) (width 0.254) (layer F.Cu) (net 8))
 (segment (start 134.575 94.125) (end 134.712999 94.262999) (width 0.254) (layer F.Cu) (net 8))
 (segment (start 134.712999 94.262999) (end 134.887961 94.262999) (width 0.254) (layer F.Cu) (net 8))
 (segment (start 134.575 94.065) (end 134.575 94.125) (width 0.254) (layer F.Cu) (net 8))
 (segment (start 125.005 101.22) (end 123.775 102.45) (width 0.254) (layer F.Cu) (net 8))
 (segment (start 127.6 101.22) (end 125.005 101.22) (width 0.254) (layer F.Cu) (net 8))
 (segment (start 133.599936 101.22) (end 135.234968 99.584968) (width 0.254) (layer F.Cu) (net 8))
 (segment (start 127.6 101.22) (end 133.599936 101.22) (width 0.254) (layer F.Cu) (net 8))
 (segment (start 135.234968 99.584968) (end 134.769936 100.05) (width 0.254) (layer F.Cu) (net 8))
 (segment (start 135.64001 99.179926) (end 135.234968 99.584968) (width 0.254) (layer F.Cu) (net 8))
 (segment (start 124.375 97.05) (end 123.675 97.75) (width 0.254) (layer F.Cu) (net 6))
 (segment (start 127.6 97.05) (end 124.375 97.05) (width 0.254) (layer F.Cu) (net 6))
 (segment (start 134.460038 94.915) (end 134.575 94.915) (width 0.254) (layer F.Cu) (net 6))
 (segment (start 133.610038 94.065) (end 134.460038 94.915) (width 0.254) (layer F.Cu) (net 6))
 (segment (start 133.225 94.065) (end 133.610038 94.065) (width 0.254) (layer F.Cu) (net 6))
 (segment (start 130.585 94.065) (end 127.6 97.05) (width 0.254) (layer F.Cu) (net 6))
 (segment (start 133.225 94.065) (end 130.585 94.065) (width 0.254) (layer F.Cu) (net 6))
 (segment (start 113.532999 104.967001) (end 120.75 97.75) (width 0.254) (layer F.Cu) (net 7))
 (segment (start 87.448399 104.967001) (end 113.532999 104.967001) (width 0.254) (layer F.Cu) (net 7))
 (segment (start 86.221398 103.74) (end 87.448399 104.967001) (width 0.254) (layer F.Cu) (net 7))
 (segment (start 80.935 103.74) (end 86.221398 103.74) (width 0.254) (layer F.Cu) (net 7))
 (segment (start 116.907999 106.392001) (end 120.85 102.45) (width 0.254) (layer F.Cu) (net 9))
 (segment (start 85.777039 106.392001) (end 116.907999 106.392001) (width 0.254) (layer F.Cu) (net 9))
 (segment (start 83.625038 104.24) (end 85.777039 106.392001) (width 0.254) (layer F.Cu) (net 9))
 (segment (start 80.935 104.24) (end 83.625038 104.24) (width 0.254) (layer F.Cu) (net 9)))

